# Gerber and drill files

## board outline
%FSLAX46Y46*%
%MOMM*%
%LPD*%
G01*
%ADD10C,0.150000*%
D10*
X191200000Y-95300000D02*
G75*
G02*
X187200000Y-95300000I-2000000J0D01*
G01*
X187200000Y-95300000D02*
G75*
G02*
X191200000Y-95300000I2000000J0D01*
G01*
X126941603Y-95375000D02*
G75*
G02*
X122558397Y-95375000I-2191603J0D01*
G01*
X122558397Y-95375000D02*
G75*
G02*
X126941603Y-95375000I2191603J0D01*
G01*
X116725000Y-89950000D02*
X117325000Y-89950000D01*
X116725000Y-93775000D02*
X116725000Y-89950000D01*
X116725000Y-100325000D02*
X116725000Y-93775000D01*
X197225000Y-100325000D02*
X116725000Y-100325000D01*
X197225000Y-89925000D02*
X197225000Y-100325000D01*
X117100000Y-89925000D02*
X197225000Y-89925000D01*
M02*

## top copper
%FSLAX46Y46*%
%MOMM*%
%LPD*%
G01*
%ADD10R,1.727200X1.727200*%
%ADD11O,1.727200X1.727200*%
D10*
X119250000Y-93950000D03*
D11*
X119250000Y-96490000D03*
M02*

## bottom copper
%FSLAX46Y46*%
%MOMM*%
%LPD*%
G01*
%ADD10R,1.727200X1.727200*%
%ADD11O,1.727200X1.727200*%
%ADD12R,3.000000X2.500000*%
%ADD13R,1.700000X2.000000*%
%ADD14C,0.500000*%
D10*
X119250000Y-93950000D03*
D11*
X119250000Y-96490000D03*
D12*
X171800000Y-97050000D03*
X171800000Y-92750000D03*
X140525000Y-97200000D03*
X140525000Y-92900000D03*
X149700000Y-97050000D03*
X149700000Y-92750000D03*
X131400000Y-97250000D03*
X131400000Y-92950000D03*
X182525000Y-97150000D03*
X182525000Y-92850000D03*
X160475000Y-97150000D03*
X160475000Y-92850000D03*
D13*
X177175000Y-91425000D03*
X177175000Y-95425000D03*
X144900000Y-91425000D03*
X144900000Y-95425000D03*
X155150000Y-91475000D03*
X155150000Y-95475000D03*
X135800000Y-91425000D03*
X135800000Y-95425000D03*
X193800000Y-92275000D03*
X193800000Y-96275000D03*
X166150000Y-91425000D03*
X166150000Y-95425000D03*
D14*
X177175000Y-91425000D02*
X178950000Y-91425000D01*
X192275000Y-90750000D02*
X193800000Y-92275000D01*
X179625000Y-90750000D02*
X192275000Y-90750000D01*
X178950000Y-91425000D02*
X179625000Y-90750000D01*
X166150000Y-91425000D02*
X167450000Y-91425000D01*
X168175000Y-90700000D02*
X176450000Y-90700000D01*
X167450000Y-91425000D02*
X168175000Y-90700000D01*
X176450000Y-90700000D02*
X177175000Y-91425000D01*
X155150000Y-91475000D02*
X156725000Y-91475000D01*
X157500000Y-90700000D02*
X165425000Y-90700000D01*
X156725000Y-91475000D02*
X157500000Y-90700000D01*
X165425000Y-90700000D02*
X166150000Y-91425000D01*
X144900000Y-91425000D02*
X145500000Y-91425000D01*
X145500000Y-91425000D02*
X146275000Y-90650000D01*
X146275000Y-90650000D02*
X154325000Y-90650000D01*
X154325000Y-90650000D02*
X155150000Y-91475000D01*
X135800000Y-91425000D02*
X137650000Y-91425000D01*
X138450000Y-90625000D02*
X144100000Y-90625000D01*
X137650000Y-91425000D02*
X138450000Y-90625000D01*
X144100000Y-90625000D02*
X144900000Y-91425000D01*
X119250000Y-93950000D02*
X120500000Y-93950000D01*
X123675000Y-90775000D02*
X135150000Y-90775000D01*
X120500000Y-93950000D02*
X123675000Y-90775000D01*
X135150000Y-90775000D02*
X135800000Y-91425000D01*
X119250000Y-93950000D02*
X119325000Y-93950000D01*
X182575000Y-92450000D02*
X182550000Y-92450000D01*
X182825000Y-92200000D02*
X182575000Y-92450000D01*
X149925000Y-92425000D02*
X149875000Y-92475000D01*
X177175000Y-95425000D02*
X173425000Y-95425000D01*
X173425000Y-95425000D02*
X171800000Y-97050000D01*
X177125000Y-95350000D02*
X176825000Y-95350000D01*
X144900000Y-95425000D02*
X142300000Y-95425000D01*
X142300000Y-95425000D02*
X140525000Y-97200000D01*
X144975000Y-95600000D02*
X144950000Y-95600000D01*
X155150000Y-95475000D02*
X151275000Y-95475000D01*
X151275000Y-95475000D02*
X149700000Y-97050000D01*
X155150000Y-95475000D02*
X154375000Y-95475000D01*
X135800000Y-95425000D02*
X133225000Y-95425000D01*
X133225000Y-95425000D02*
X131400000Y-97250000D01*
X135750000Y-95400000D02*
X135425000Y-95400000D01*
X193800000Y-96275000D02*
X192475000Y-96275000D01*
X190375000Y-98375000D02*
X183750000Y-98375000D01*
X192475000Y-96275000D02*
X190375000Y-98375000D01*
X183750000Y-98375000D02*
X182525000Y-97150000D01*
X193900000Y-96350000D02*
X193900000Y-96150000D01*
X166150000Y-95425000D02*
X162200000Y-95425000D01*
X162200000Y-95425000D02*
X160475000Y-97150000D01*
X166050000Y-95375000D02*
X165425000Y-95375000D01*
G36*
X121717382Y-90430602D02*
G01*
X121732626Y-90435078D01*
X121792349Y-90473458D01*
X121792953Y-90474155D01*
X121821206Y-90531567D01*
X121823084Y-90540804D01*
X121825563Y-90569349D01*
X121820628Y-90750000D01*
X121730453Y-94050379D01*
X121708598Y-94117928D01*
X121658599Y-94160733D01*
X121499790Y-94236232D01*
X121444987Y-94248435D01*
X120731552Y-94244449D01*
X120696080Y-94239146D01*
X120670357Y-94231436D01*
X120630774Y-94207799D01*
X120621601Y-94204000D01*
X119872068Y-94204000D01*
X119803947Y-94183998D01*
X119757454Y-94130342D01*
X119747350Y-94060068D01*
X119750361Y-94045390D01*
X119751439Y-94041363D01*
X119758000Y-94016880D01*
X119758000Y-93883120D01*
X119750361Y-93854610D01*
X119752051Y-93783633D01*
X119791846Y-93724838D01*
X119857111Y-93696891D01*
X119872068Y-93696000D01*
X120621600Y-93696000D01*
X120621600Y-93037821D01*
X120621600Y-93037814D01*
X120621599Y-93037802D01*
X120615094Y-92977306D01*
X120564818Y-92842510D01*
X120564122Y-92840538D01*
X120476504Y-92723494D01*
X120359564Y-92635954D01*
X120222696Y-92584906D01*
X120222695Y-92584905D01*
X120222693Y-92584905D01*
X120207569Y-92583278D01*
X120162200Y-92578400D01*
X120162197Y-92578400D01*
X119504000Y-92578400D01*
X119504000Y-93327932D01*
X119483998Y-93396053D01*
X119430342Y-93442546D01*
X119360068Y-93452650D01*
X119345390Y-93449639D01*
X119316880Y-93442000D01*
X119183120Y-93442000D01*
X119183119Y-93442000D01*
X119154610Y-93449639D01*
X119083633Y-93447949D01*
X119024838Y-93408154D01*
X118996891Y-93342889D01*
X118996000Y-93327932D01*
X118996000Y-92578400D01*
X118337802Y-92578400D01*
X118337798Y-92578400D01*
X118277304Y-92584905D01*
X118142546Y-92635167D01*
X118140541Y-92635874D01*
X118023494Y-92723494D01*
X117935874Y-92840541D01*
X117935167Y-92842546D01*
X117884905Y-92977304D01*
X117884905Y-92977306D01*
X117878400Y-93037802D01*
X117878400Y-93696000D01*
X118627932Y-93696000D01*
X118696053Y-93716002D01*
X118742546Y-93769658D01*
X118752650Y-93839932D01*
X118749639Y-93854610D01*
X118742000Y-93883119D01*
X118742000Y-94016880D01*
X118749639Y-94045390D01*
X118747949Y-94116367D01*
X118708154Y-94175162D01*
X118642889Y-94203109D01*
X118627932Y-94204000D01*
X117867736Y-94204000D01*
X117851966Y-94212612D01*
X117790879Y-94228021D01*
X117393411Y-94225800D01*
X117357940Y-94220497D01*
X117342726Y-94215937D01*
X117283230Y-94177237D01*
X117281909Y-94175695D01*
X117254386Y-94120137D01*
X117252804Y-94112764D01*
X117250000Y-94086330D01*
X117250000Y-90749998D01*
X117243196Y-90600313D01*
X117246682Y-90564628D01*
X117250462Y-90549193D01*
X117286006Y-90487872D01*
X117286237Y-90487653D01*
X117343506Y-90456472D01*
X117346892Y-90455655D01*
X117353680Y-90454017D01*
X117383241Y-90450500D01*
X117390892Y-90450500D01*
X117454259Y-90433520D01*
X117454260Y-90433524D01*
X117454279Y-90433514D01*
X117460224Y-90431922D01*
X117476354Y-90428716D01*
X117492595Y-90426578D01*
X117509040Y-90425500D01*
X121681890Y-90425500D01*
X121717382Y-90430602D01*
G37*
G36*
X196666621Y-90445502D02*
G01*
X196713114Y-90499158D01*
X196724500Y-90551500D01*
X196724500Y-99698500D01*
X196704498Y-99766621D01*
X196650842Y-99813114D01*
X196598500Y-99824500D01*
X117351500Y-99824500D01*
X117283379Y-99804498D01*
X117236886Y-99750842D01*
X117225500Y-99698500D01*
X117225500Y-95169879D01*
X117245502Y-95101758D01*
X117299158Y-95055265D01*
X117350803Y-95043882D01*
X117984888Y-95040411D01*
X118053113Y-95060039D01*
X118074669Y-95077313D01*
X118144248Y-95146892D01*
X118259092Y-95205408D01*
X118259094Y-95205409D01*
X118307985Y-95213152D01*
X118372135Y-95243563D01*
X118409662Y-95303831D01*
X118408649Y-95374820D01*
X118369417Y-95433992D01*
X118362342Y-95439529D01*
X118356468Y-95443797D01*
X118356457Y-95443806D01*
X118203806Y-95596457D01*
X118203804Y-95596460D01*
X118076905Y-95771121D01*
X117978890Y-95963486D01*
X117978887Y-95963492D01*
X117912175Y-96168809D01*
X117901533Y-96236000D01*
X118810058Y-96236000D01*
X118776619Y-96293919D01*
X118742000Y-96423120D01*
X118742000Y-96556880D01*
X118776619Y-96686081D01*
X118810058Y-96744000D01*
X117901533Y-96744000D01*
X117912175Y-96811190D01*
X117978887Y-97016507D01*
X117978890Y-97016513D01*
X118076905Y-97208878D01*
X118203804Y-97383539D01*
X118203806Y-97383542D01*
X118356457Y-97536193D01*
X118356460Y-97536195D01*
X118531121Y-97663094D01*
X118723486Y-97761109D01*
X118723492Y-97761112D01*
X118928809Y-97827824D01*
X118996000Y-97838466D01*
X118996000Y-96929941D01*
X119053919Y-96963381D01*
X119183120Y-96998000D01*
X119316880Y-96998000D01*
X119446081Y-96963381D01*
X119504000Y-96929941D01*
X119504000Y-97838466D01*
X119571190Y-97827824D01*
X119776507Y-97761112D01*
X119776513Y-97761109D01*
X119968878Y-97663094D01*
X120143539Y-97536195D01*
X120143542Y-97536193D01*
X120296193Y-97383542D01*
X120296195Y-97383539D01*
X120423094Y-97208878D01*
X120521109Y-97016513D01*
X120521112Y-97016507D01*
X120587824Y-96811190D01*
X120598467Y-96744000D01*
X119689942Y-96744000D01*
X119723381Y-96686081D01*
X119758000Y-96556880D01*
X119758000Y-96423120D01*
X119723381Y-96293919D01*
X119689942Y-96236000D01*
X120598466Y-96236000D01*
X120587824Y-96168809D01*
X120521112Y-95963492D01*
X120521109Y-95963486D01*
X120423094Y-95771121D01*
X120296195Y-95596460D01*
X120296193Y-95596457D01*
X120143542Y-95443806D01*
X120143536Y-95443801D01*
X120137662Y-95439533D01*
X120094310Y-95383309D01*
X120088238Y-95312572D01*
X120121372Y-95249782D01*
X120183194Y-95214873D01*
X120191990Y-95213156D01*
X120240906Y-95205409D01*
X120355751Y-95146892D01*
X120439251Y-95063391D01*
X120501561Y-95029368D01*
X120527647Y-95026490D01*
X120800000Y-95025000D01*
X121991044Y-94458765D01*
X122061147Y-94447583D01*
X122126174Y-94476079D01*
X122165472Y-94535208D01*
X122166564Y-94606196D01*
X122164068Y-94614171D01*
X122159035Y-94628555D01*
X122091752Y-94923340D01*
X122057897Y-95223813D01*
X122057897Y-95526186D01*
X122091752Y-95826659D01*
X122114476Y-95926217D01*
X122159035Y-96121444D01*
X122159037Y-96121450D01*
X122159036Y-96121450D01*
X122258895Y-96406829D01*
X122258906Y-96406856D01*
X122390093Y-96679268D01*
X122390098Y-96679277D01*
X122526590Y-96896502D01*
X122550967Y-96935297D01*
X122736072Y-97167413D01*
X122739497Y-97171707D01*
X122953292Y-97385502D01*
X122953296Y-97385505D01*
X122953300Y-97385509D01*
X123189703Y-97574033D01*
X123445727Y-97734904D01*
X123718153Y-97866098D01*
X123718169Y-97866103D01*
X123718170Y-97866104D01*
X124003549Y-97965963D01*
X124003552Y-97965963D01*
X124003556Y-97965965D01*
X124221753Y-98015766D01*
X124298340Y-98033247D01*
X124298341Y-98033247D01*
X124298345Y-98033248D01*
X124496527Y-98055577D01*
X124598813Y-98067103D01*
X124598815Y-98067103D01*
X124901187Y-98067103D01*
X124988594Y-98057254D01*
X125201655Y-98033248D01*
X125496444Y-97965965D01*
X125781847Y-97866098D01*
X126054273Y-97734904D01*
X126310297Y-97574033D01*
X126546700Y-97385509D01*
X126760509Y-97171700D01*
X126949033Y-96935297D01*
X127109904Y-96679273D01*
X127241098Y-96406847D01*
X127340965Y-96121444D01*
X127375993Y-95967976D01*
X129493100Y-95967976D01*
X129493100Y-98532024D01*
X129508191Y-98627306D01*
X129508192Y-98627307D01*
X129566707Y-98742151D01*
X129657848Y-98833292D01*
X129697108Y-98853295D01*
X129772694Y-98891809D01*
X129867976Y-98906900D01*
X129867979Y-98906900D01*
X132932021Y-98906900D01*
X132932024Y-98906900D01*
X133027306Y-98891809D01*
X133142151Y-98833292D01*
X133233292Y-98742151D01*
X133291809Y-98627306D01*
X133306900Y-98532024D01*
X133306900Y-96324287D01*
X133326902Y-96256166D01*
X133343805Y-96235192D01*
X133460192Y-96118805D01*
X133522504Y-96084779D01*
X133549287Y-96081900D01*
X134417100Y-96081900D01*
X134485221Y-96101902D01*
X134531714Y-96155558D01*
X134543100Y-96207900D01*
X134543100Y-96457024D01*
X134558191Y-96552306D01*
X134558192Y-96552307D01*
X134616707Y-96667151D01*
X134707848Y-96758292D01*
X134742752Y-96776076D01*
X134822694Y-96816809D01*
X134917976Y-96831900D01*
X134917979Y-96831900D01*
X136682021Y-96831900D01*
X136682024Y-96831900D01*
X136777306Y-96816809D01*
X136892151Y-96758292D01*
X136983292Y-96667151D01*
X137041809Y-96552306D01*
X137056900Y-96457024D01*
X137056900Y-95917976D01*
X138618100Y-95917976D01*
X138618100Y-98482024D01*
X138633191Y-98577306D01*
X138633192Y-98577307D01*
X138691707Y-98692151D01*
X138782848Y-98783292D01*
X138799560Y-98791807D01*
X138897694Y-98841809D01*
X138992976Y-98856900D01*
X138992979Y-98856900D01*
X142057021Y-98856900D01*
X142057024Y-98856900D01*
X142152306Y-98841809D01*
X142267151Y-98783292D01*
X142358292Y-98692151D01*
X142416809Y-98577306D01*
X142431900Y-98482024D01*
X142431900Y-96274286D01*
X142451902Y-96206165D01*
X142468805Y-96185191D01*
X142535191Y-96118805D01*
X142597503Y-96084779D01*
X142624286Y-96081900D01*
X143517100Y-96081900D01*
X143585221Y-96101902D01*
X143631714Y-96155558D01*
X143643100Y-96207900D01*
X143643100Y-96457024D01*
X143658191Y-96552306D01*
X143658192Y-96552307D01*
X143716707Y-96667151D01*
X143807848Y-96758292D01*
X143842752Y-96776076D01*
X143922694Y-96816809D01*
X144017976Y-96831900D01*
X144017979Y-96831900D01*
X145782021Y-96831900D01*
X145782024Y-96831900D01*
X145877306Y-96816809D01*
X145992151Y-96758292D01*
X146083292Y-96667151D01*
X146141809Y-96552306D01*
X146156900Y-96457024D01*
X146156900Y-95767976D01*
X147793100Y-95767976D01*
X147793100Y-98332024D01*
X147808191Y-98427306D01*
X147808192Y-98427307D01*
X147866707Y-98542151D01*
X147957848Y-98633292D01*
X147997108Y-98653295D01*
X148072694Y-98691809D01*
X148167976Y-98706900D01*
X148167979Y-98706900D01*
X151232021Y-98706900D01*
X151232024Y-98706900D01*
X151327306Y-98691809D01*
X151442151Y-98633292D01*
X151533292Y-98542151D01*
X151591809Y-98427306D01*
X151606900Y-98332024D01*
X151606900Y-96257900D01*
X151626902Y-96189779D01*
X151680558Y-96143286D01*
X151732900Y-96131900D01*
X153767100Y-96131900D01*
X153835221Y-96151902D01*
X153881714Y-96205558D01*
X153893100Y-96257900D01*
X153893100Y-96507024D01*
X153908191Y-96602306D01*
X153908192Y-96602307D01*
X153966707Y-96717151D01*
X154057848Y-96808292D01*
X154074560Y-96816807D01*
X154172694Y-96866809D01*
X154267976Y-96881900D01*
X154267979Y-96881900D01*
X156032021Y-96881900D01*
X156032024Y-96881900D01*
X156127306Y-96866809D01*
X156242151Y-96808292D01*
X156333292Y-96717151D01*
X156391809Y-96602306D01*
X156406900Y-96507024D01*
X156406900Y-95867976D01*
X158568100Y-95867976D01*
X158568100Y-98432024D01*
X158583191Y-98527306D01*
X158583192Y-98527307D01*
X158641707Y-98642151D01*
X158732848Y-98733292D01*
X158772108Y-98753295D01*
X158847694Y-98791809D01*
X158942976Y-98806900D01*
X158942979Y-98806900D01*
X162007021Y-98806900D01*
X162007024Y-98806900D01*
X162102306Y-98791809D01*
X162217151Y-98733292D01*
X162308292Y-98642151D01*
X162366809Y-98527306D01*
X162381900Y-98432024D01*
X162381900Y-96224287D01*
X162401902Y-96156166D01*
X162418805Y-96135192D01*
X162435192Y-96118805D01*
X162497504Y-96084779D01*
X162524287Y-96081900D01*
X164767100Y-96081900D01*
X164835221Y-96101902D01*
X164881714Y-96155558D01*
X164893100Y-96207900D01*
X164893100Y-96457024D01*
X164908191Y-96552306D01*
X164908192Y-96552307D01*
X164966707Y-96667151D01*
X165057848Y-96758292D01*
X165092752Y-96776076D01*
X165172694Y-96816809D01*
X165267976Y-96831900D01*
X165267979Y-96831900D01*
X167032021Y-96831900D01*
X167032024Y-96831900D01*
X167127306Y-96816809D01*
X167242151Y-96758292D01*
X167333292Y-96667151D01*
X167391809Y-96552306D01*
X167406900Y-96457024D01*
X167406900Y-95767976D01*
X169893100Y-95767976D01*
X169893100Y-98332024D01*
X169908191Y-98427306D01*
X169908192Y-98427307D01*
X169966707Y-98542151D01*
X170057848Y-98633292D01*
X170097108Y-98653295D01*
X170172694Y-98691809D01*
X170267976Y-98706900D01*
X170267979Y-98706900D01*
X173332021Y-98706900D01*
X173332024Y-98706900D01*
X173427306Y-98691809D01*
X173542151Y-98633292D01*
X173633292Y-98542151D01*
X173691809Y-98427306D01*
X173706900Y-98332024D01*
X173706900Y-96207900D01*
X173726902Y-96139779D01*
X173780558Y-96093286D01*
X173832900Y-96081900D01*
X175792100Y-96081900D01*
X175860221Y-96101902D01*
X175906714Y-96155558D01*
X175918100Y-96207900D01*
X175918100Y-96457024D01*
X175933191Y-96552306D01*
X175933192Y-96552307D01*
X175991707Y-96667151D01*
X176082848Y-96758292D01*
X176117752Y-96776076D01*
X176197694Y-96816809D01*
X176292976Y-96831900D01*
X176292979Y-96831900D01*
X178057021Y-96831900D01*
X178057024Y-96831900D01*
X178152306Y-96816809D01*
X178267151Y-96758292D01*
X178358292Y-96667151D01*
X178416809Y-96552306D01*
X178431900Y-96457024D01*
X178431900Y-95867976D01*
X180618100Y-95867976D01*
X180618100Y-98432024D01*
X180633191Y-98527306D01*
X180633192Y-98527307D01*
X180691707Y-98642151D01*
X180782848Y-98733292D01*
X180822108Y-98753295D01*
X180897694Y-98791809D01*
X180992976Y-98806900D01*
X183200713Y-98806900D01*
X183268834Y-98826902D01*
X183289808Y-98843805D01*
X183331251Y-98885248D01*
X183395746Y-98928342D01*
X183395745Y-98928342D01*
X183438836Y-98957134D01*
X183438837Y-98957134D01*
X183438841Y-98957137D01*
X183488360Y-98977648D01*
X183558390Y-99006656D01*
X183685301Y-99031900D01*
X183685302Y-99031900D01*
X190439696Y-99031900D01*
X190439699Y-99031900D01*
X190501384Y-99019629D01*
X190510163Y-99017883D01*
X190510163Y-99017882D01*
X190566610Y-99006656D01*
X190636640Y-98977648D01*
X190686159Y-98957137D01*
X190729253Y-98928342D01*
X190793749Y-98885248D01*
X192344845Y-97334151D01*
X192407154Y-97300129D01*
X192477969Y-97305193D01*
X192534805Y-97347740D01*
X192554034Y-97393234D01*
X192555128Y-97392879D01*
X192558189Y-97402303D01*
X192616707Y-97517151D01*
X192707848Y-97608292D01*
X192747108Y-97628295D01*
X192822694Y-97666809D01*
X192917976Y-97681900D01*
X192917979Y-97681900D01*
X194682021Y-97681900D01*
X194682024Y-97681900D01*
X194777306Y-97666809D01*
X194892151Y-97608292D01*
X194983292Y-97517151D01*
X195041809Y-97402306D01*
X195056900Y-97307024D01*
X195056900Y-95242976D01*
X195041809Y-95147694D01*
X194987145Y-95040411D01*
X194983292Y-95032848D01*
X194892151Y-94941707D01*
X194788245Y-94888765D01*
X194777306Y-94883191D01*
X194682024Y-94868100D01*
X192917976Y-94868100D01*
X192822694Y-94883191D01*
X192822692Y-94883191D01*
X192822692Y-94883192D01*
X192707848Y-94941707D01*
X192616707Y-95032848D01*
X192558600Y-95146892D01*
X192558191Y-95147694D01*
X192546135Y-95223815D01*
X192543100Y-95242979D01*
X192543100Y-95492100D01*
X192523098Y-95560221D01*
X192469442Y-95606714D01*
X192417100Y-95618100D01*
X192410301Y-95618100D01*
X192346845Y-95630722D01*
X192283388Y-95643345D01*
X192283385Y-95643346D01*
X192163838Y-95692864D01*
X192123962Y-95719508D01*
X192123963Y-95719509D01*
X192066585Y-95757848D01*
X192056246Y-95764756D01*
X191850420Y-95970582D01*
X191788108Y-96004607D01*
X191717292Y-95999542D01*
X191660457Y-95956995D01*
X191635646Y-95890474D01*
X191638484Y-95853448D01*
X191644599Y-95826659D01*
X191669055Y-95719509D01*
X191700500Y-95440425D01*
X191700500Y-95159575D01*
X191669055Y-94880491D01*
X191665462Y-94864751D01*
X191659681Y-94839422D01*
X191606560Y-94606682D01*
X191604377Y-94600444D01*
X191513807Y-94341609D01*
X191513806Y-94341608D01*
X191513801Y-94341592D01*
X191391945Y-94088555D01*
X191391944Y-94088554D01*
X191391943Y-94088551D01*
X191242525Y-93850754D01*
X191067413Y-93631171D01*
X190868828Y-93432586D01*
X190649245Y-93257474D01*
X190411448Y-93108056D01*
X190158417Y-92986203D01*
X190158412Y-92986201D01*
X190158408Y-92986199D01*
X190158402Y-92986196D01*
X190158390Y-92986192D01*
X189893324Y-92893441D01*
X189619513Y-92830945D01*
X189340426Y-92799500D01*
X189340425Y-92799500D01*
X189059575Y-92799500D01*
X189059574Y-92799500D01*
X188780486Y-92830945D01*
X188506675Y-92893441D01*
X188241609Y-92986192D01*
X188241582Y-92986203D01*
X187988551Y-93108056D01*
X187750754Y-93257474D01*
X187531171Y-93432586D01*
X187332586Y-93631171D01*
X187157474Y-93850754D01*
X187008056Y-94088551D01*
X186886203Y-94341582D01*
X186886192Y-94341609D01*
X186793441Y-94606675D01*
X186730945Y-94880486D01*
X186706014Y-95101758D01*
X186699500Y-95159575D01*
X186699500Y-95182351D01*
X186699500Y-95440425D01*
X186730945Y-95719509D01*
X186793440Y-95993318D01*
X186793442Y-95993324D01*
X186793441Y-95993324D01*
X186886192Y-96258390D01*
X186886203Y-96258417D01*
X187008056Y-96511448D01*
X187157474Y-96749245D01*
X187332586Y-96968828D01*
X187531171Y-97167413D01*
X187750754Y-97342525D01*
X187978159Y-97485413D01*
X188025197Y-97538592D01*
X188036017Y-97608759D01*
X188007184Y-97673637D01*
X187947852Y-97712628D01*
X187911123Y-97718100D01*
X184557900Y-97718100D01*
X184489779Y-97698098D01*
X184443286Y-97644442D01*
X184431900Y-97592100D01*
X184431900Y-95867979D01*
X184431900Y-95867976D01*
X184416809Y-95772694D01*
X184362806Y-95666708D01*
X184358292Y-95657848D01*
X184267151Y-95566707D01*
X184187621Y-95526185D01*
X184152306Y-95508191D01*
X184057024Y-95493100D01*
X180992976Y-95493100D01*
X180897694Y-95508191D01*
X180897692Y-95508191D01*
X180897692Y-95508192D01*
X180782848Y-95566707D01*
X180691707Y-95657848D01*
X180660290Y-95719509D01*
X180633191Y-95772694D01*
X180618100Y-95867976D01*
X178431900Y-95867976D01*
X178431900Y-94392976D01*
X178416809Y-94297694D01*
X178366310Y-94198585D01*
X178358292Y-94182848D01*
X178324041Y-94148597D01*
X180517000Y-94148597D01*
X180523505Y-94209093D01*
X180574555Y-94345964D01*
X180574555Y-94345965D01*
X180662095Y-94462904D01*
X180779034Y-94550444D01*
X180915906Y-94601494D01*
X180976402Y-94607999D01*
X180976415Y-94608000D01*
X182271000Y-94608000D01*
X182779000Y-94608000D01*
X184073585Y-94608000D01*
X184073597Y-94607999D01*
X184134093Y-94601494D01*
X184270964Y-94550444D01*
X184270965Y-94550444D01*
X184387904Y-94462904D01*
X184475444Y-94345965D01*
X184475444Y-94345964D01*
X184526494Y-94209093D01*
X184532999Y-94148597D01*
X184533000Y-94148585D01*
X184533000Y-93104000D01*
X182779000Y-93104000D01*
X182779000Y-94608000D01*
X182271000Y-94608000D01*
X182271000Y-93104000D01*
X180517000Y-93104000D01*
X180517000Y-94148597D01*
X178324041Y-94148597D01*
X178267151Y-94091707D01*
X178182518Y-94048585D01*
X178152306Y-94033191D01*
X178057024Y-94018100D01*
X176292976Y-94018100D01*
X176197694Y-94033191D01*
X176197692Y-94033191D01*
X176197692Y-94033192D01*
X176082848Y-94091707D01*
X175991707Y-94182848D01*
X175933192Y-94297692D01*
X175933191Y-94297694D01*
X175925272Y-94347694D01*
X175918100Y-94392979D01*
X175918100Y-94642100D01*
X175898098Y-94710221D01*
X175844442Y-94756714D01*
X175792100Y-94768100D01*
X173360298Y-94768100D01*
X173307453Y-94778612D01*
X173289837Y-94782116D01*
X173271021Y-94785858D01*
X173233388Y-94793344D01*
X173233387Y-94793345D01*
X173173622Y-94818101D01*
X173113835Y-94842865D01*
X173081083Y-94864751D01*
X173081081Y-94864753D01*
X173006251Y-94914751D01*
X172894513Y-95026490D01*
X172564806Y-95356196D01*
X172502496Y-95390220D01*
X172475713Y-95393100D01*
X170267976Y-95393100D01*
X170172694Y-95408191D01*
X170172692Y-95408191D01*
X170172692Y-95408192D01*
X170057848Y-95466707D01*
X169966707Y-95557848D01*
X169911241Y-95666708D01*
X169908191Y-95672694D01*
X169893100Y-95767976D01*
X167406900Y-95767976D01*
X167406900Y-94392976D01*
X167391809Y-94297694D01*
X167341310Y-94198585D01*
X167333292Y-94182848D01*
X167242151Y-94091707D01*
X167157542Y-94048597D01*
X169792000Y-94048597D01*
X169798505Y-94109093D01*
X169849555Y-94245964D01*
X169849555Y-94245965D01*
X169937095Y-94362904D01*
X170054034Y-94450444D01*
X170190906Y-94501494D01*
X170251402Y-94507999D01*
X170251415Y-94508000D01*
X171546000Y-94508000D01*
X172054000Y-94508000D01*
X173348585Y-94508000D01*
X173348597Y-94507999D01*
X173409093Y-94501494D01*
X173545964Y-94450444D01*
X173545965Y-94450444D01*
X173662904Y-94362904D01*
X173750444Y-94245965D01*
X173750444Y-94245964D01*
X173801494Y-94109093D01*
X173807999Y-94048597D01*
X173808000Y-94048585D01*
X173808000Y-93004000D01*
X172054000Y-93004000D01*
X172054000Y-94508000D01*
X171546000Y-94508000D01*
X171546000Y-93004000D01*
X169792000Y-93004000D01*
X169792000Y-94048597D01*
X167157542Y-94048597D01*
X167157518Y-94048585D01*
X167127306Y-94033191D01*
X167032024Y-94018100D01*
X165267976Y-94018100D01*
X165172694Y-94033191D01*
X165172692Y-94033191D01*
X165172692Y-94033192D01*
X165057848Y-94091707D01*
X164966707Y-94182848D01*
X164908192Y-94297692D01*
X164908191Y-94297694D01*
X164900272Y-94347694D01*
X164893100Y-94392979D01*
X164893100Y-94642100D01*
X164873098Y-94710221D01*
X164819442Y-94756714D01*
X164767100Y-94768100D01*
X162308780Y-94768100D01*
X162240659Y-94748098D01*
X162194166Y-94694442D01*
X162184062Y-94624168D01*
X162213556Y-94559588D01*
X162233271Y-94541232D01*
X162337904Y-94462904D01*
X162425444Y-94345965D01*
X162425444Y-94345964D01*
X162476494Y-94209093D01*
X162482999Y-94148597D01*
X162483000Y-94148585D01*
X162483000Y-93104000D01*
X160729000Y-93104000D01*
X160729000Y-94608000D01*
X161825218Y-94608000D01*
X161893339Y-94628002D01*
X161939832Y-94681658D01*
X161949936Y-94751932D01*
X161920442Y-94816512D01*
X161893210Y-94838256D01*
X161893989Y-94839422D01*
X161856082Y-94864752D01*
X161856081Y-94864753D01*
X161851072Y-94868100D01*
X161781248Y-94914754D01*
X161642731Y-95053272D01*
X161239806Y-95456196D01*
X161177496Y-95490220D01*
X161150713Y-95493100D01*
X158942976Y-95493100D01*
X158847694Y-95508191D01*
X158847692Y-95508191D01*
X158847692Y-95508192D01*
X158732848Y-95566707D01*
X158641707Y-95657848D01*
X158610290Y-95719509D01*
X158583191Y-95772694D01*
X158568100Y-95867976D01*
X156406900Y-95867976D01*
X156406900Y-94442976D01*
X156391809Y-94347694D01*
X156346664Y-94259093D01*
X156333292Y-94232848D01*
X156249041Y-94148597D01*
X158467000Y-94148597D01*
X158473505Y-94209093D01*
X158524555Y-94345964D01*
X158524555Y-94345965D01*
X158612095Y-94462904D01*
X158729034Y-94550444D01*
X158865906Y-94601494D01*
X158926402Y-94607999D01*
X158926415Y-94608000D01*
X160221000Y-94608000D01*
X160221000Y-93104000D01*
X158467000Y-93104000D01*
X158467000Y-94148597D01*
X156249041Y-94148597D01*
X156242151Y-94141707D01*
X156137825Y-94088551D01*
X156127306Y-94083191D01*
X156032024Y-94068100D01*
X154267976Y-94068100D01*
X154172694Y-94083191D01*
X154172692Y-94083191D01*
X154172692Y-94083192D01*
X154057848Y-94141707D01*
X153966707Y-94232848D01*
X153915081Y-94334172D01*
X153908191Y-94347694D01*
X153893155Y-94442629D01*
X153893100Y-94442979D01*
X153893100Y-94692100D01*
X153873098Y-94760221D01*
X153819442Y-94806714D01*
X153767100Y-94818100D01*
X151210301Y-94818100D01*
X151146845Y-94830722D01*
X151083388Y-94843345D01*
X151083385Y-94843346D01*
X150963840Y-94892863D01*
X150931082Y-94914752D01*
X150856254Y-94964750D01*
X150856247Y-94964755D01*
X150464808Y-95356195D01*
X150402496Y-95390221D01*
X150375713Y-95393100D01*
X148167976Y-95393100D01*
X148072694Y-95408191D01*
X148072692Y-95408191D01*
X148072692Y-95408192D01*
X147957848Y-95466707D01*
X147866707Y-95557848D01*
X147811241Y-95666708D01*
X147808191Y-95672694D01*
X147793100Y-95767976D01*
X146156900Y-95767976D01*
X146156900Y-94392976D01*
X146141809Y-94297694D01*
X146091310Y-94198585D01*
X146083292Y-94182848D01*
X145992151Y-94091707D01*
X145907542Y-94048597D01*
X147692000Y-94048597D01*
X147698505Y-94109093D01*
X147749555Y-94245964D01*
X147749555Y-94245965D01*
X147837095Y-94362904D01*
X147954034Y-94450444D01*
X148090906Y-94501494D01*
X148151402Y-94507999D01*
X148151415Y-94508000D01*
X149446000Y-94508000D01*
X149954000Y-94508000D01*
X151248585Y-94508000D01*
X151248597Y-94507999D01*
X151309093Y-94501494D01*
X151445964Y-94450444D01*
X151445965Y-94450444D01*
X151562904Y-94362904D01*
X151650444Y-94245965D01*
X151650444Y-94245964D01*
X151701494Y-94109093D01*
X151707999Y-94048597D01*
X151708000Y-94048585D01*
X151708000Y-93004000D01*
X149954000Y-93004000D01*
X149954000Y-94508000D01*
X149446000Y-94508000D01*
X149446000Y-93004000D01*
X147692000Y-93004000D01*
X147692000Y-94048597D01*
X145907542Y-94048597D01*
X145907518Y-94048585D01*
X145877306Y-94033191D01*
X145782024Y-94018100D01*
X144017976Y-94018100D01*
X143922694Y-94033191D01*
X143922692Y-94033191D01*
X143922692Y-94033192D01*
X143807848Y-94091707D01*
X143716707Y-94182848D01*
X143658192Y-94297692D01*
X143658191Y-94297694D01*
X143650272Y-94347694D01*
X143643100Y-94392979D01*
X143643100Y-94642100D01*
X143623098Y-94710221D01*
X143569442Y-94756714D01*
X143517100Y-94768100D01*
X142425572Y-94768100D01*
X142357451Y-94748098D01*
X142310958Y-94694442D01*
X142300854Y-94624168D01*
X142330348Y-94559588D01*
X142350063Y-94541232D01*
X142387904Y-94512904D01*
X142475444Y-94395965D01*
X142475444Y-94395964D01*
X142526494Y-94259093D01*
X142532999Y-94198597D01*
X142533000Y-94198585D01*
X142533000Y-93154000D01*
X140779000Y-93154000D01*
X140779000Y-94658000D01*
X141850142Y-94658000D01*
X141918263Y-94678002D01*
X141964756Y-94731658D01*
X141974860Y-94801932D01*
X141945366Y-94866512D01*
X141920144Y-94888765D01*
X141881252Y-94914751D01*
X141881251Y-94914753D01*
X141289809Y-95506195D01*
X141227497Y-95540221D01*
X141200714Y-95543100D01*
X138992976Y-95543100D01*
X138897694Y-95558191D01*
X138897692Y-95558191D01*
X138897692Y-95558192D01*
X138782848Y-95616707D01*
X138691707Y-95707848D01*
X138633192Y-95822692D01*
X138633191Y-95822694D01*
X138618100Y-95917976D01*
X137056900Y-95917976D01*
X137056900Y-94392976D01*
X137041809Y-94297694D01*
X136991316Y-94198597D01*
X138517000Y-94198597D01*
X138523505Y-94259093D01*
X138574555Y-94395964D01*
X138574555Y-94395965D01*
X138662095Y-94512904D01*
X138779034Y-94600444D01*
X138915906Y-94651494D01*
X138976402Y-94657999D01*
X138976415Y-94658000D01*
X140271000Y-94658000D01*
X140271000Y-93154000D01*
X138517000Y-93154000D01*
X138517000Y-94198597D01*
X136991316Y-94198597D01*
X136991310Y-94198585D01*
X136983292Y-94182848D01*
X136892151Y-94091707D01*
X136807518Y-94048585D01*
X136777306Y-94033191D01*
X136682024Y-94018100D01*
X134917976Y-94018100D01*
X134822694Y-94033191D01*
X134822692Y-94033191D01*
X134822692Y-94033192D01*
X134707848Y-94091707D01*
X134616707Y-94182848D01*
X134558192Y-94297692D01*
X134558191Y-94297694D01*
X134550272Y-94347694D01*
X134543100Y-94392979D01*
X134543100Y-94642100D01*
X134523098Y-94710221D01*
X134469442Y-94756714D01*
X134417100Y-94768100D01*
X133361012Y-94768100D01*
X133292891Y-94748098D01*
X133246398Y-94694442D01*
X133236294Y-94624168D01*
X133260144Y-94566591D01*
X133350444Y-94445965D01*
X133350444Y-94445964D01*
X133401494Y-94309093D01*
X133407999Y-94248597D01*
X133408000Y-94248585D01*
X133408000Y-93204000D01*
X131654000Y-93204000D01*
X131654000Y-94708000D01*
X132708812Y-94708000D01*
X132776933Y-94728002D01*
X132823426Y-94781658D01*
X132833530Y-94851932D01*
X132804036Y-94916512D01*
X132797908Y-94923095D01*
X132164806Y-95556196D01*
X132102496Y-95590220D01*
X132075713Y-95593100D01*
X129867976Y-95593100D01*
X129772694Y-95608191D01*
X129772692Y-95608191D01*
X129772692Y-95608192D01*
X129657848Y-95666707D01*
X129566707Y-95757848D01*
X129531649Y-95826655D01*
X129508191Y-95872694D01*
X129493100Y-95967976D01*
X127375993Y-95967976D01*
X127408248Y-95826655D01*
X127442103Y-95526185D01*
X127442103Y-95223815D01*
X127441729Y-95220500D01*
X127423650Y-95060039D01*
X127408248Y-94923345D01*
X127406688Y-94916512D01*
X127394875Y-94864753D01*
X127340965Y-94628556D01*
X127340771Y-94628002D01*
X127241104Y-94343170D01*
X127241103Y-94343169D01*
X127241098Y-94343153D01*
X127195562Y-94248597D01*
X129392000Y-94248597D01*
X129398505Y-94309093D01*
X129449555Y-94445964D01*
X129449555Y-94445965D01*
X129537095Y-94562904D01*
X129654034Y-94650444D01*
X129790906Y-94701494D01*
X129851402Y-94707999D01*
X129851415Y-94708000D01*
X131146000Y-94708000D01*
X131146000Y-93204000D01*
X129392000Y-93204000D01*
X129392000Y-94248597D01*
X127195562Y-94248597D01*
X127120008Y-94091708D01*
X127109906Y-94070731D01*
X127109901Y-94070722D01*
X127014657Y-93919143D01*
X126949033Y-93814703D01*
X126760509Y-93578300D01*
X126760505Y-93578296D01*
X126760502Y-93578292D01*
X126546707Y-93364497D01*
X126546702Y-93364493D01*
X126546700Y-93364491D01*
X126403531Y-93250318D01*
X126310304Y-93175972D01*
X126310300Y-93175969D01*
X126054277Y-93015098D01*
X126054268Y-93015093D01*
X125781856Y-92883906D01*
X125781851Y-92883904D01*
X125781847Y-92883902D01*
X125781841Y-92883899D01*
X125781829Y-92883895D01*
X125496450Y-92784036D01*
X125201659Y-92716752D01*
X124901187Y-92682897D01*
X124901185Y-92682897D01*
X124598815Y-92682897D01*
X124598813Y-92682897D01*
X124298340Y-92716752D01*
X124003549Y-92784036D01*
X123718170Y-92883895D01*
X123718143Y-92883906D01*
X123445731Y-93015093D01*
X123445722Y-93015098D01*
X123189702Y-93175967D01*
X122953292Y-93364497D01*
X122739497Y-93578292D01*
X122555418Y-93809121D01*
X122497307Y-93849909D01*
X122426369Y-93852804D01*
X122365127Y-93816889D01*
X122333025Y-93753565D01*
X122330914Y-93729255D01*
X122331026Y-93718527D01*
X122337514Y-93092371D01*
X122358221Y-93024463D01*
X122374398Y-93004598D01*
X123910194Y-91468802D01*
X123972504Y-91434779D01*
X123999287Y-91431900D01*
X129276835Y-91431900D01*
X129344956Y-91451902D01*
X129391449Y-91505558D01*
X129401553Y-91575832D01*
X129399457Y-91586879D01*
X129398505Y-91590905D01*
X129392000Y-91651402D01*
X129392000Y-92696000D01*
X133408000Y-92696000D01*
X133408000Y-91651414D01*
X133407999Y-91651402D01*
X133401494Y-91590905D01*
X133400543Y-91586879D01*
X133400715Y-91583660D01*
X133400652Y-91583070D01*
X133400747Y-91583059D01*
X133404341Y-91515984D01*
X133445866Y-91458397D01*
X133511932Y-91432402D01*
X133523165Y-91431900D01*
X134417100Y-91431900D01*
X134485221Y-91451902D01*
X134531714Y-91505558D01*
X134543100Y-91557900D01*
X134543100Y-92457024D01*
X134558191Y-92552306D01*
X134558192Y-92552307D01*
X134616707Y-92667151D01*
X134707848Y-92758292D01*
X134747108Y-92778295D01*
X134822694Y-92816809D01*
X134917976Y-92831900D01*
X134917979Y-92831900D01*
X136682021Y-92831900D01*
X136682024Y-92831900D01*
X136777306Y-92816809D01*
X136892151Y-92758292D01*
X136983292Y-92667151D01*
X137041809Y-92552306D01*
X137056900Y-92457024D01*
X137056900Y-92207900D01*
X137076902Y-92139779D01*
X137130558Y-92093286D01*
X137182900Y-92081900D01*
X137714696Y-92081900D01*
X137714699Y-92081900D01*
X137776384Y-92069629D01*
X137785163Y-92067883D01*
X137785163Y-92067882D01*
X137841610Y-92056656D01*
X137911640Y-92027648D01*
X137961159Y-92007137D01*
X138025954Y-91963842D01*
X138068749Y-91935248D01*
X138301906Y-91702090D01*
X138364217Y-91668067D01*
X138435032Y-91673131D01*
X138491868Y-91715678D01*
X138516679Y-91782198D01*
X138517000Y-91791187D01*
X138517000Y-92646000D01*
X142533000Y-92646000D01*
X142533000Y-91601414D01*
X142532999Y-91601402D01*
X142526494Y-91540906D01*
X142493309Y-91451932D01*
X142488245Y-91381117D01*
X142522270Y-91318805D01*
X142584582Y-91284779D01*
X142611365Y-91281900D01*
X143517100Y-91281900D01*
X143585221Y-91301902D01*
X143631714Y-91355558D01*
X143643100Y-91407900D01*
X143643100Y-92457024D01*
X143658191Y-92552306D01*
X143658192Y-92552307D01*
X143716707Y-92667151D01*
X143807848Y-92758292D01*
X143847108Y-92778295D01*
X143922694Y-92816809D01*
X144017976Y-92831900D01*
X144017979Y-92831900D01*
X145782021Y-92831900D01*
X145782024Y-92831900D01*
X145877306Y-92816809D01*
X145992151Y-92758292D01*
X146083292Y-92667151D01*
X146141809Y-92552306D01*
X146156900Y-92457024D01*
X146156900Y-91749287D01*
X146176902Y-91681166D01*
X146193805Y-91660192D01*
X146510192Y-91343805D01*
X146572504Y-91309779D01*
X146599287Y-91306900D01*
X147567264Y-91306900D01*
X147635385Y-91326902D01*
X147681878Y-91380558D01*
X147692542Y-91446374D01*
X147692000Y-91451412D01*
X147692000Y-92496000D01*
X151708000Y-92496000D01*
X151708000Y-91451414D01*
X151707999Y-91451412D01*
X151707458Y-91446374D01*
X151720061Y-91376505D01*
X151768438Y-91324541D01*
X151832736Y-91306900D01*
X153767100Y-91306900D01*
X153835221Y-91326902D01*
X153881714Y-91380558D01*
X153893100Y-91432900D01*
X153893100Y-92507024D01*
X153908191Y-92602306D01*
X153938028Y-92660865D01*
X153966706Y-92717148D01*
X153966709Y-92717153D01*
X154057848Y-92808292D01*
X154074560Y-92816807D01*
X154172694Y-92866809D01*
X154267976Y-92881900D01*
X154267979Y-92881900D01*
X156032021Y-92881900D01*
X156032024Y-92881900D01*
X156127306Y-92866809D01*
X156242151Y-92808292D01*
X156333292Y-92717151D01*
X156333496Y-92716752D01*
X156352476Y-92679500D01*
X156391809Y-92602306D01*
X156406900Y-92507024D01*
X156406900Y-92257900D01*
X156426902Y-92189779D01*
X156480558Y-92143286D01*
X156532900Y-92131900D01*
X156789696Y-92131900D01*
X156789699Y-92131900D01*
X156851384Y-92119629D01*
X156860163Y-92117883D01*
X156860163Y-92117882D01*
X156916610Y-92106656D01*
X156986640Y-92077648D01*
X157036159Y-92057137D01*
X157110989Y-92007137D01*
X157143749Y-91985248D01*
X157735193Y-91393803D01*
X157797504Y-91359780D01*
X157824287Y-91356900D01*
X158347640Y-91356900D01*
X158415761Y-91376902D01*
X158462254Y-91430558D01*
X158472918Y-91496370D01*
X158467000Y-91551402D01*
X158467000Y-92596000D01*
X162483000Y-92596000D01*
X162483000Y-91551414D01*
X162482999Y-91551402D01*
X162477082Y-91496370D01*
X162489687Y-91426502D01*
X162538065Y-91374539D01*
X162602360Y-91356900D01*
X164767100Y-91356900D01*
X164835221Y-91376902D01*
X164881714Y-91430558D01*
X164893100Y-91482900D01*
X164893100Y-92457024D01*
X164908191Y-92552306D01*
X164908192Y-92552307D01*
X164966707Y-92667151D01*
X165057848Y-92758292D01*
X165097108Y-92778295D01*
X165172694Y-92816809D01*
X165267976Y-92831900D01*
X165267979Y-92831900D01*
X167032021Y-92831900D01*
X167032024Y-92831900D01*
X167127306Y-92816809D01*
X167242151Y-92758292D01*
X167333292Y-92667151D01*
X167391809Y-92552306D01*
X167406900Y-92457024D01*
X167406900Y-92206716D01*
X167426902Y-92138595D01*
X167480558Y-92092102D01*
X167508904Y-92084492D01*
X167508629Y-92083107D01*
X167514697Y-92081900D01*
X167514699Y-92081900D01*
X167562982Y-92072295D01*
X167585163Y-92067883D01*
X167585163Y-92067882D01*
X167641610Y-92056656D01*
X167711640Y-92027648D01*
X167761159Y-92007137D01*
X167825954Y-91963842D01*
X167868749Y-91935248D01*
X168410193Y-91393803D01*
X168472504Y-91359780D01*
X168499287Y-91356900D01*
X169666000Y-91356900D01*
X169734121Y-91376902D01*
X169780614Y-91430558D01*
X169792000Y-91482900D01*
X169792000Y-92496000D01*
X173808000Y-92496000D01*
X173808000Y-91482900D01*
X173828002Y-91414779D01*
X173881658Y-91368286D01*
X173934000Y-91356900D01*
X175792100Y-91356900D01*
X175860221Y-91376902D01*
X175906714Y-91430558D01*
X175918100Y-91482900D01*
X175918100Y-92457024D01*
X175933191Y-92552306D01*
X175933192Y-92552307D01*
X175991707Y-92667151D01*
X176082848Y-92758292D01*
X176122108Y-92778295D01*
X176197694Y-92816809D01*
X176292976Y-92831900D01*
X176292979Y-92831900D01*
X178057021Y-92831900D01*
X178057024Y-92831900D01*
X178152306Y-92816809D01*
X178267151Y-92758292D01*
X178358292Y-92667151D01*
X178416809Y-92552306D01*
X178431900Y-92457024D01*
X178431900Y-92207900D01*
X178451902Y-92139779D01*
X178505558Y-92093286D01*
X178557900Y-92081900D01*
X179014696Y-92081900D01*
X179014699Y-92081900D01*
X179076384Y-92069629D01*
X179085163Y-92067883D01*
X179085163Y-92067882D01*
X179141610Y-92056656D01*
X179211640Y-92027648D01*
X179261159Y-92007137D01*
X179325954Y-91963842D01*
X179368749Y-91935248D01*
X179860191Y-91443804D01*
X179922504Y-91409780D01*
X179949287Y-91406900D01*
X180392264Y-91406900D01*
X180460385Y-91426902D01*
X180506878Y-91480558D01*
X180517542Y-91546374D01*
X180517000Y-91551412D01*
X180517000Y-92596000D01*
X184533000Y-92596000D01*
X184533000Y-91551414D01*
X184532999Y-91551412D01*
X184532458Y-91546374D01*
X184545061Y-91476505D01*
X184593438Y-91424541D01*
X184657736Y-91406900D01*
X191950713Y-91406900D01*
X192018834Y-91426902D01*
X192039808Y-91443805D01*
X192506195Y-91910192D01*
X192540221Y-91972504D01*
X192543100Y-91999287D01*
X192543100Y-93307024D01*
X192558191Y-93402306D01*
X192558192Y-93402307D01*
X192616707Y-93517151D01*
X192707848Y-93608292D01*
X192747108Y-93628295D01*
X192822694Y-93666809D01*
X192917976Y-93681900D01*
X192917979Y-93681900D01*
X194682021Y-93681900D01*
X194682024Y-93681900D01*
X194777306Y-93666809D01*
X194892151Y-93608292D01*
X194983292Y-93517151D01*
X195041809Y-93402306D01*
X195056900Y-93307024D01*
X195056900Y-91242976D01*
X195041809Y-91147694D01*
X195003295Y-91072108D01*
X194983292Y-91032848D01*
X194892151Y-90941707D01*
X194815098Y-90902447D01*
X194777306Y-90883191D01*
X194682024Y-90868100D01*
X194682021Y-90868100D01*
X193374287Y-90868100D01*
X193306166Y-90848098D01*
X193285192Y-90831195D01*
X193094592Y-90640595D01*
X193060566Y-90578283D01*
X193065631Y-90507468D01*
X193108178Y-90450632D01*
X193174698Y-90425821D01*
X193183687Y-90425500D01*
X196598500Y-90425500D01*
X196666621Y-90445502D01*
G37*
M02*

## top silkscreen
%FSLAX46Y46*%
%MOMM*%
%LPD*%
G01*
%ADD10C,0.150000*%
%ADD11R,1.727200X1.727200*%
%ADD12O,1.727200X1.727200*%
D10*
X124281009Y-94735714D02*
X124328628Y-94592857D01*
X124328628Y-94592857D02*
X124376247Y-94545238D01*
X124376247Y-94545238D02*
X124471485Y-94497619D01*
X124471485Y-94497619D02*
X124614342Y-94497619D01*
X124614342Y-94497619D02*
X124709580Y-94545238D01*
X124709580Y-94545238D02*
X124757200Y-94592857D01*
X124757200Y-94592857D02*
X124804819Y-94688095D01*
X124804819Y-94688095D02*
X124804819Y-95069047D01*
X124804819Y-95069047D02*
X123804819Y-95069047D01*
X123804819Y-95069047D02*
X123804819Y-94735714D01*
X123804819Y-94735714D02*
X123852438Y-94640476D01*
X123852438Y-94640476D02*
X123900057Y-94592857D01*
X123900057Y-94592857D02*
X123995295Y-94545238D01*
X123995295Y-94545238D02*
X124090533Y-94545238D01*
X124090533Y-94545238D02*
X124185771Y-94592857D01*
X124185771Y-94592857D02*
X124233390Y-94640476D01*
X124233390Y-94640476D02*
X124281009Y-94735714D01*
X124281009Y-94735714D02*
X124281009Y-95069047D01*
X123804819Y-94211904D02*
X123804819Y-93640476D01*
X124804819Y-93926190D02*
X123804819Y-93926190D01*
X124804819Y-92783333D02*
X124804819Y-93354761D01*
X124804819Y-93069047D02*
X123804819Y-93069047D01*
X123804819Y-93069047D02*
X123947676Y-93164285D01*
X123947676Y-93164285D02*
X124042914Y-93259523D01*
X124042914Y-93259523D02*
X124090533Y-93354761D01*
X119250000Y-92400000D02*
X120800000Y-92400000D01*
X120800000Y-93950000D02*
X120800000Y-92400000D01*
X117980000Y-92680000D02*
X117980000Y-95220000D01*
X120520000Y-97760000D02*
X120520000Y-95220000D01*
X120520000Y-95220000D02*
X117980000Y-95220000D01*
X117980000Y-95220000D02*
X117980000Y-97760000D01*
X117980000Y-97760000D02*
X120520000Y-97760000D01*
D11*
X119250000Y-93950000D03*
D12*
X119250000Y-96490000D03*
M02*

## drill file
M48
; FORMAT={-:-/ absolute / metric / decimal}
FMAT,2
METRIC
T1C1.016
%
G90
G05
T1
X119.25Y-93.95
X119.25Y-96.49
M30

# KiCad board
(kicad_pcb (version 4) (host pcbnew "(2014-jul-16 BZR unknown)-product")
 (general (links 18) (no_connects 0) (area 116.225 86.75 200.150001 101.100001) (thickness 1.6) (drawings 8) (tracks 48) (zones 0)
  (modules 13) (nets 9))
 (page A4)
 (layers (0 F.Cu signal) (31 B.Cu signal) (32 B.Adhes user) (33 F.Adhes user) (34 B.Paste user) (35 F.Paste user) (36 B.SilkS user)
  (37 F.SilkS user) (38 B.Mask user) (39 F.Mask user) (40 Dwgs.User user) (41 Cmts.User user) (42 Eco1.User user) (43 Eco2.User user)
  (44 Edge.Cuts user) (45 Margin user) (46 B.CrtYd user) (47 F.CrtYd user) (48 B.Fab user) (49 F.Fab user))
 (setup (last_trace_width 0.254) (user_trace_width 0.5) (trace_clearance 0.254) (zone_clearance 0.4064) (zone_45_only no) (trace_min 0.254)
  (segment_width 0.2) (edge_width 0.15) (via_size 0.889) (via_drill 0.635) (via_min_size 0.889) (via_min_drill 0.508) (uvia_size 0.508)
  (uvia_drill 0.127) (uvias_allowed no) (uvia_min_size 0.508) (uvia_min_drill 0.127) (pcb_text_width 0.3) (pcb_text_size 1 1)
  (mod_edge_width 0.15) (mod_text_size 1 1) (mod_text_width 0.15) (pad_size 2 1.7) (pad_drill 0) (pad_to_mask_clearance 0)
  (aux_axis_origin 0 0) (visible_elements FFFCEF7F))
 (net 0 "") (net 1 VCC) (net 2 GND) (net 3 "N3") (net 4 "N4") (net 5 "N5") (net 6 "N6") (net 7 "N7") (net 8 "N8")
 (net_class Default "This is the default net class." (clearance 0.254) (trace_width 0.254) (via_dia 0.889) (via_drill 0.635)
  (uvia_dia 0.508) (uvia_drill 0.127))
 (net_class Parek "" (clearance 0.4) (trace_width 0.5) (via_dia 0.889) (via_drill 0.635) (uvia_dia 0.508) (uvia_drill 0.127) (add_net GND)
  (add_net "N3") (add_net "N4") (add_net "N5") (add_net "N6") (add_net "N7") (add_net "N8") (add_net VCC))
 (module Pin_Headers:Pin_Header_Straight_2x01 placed (layer F.Cu) (at 119.25 93.95 270)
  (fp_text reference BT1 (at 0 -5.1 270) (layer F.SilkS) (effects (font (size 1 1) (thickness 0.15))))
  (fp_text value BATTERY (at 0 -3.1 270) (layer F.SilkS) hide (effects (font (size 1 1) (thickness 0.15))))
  (fp_line (start -1.55 0) (end -1.55 -1.55) (layer F.SilkS) (width 0.15))
  (fp_line (start 0 -1.55) (end -1.55 -1.55) (layer F.SilkS) (width 0.15))
  (fp_line (start -1.27 1.27) (end 1.27 1.27) (layer F.SilkS) (width 0.15))
  (fp_line (start 3.81 -1.27) (end 1.27 -1.27) (layer F.SilkS) (width 0.15))
  (fp_line (start 1.27 -1.27) (end 1.27 1.27) (layer F.SilkS) (width 0.15))
  (fp_line (start 1.27 1.27) (end 3.81 1.27) (layer F.SilkS) (width 0.15))
  (fp_line (start 3.81 1.27) (end 3.81 -1.27) (layer F.SilkS) (width 0.15))
  (pad 1 thru_hole rect (at 0 0 270) (size 1.7272 1.7272) (drill 1.016) (layers *.Cu *.Mask F.SilkS) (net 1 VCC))
  (pad 2 thru_hole oval (at 2.54 0 270) (size 1.7272 1.7272) (drill 1.016) (layers *.Cu *.Mask F.SilkS) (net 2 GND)))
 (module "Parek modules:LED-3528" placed (layer B.Cu) (at 171.8 94.9 90)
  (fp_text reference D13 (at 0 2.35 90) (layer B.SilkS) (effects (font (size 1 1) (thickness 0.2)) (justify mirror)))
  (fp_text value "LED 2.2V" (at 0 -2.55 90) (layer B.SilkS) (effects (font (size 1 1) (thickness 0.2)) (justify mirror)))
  (pad 1 smd rect (at -2.15 0 90) (size 2.5 3) (layers B.Cu B.Paste B.Mask) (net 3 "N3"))
  (pad 2 smd rect (at 2.15 0 90) (size 2.5 3) (layers B.Cu B.Paste B.Mask) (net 2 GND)))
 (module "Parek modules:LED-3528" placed (layer B.Cu) (at 140.525 95.05 90)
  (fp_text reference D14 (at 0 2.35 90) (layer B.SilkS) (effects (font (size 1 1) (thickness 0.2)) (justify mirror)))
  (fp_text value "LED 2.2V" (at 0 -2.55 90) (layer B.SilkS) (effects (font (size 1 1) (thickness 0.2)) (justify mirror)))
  (pad 1 smd rect (at -2.15 0 90) (size 2.5 3) (layers B.Cu B.Paste B.Mask) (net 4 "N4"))
  (pad 2 smd rect (at 2.15 0 90) (size 2.5 3) (layers B.Cu B.Paste B.Mask) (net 2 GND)))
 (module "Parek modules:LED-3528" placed (layer B.Cu) (at 149.7 94.9 90)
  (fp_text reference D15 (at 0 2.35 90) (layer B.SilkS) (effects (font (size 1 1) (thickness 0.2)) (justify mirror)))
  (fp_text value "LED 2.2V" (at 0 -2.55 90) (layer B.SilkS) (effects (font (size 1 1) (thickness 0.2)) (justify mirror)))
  (pad 1 smd rect (at -2.15 0 90) (size 2.5 3) (layers B.Cu B.Paste B.Mask) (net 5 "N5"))
  (pad 2 smd rect (at 2.15 0 90) (size 2.5 3) (layers B.Cu B.Paste B.Mask) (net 2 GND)))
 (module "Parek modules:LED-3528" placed (layer B.Cu) (at 131.4 95.1 90)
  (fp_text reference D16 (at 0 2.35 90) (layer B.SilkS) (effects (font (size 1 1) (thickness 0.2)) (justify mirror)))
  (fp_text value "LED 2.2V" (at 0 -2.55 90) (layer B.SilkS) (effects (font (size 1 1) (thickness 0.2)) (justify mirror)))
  (pad 1 smd rect (at -2.15 0 90) (size 2.5 3) (layers B.Cu B.Paste B.Mask) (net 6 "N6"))
  (pad 2 smd rect (at 2.15 0 90) (size 2.5 3) (layers B.Cu B.Paste B.Mask) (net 2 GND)))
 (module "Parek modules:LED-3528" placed (layer B.Cu) (at 182.525 95 90)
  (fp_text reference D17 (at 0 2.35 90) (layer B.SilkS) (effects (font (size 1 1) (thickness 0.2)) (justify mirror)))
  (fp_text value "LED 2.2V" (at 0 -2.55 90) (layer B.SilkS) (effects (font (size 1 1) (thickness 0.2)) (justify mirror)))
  (pad 1 smd rect (at -2.15 0 90) (size 2.5 3) (layers B.Cu B.Paste B.Mask) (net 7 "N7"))
  (pad 2 smd rect (at 2.15 0 90) (size 2.5 3) (layers B.Cu B.Paste B.Mask) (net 2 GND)))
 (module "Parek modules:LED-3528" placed (layer B.Cu) (at 160.475 95 90)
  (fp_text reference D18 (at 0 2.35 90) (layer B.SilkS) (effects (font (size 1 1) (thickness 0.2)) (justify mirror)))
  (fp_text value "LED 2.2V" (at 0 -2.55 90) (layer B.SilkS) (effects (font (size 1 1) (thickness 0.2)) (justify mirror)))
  (pad 1 smd rect (at -2.15 0 90) (size 2.5 3) (layers B.Cu B.Paste B.Mask) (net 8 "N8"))
  (pad 2 smd rect (at 2.15 0 90) (size 2.5 3) (layers B.Cu B.Paste B.Mask) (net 2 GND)))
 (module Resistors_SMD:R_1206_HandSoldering (layer B.Cu) (at 177.175 93.425 270)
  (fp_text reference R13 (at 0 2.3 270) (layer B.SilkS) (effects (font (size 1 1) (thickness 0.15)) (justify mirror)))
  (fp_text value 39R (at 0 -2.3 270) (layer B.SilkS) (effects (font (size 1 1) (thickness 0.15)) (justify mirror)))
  (pad 1 smd rect (at -2 0 270) (size 2 1.7) (layers B.Cu B.Paste B.Mask) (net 1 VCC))
  (pad 2 smd rect (at 2 0 270) (size 2 1.7) (layers B.Cu B.Paste B.Mask) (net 3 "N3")))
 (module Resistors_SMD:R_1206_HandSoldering (layer B.Cu) (at 144.9 93.425 270)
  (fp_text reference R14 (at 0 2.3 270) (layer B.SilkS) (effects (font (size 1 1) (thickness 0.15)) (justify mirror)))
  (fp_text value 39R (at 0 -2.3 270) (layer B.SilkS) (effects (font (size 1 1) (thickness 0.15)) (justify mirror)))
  (pad 1 smd rect (at -2 0 270) (size 2 1.7) (layers B.Cu B.Paste B.Mask) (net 1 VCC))
  (pad 2 smd rect (at 2 0 270) (size 2 1.7) (layers B.Cu B.Paste B.Mask) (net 4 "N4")))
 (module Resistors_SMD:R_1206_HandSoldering (layer B.Cu) (at 155.15 93.475 270)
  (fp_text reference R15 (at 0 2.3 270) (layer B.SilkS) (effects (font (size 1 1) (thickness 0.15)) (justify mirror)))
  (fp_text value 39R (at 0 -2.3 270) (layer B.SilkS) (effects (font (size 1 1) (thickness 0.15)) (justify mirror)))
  (pad 1 smd rect (at -2 0 270) (size 2 1.7) (layers B.Cu B.Paste B.Mask) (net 1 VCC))
  (pad 2 smd rect (at 2 0 270) (size 2 1.7) (layers B.Cu B.Paste B.Mask) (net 5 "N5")))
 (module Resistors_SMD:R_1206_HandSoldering (layer B.Cu) (at 135.8 93.425 270)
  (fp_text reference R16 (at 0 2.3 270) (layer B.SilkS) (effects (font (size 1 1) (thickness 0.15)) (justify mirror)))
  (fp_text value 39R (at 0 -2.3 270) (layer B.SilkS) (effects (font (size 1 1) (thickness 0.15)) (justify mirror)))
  (pad 1 smd rect (at -2 0 270) (size 2 1.7) (layers B.Cu B.Paste B.Mask) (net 1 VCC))
  (pad 2 smd rect (at 2 0 270) (size 2 1.7) (layers B.Cu B.Paste B.Mask) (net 6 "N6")))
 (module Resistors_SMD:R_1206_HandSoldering (layer B.Cu) (at 193.8 94.275 270)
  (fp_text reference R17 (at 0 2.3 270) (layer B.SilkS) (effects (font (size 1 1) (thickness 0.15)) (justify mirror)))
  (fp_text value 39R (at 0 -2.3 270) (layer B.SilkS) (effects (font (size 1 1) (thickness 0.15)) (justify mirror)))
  (pad 1 smd rect (at -2 0 270) (size 2 1.7) (layers B.Cu B.Paste B.Mask) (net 1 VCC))
  (pad 2 smd rect (at 2 0 270) (size 2 1.7) (layers B.Cu B.Paste B.Mask) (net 7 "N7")))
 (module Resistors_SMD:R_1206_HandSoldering (layer B.Cu) (at 166.15 93.425 270)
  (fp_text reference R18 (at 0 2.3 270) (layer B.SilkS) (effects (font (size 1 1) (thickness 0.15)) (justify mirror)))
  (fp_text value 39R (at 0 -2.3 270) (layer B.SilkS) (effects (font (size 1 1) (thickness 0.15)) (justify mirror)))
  (pad 1 smd rect (at -2 0 270) (size 2 1.7) (layers B.Cu B.Paste B.Mask) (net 1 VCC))
  (pad 2 smd rect (at 2 0 270) (size 2 1.7) (layers B.Cu B.Paste B.Mask) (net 8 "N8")))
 (gr_circle (center 189.2 95.3) (end 189.2 97.3) (layer Edge.Cuts) (width 0.15))
 (gr_circle (center 124.75 95.375) (end 125.7 97.35) (layer Edge.Cuts) (width 0.15))
 (gr_line (start 116.725 89.95) (end 117.325 89.95) (angle 90) (layer Edge.Cuts) (width 0.15))
 (gr_line (start 116.725 93.775) (end 116.725 89.95) (angle 90) (layer Edge.Cuts) (width 0.15))
 (gr_line (start 116.725 100.325) (end 116.725 93.775) (angle 90) (layer Edge.Cuts) (width 0.15))
 (gr_line (start 197.225 100.325) (end 116.725 100.325) (angle 90) (layer Edge.Cuts) (width 0.15))
 (gr_line (start 197.225 89.925) (end 197.225 100.325) (angle 90) (layer Edge.Cuts) (width 0.15))
 (gr_line (start 117.1 89.925) (end 197.225 89.925) (angle 90) (layer Edge.Cuts) (width 0.15))
 (segment (start 177.175 91.425) (end 178.95 91.425) (width 0.5) (layer B.Cu) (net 1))
 (segment (start 192.275 90.75) (end 193.8 92.275) (width 0.5) (layer B.Cu) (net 1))
 (segment (start 179.625 90.75) (end 192.275 90.75) (width 0.5) (layer B.Cu) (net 1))
 (segment (start 178.95 91.425) (end 179.625 90.75) (width 0.5) (layer B.Cu) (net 1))
 (segment (start 166.15 91.425) (end 167.45 91.425) (width 0.5) (layer B.Cu) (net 1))
 (segment (start 168.175 90.7) (end 176.45 90.7) (width 0.5) (layer B.Cu) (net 1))
 (segment (start 167.45 91.425) (end 168.175 90.7) (width 0.5) (layer B.Cu) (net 1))
 (segment (start 176.45 90.7) (end 177.175 91.425) (width 0.5) (layer B.Cu) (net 1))
 (segment (start 155.15 91.475) (end 156.725 91.475) (width 0.5) (layer B.Cu) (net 1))
 (segment (start 157.5 90.7) (end 165.425 90.7) (width 0.5) (layer B.Cu) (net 1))
 (segment (start 156.725 91.475) (end 157.5 90.7) (width 0.5) (layer B.Cu) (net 1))
 (segment (start 165.425 90.7) (end 166.15 91.425) (width 0.5) (layer B.Cu) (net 1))
 (segment (start 144.9 91.425) (end 145.5 91.425) (width 0.5) (layer B.Cu) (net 1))
 (segment (start 145.5 91.425) (end 146.275 90.65) (width 0.5) (layer B.Cu) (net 1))
 (segment (start 146.275 90.65) (end 154.325 90.65) (width 0.5) (layer B.Cu) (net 1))
 (segment (start 154.325 90.65) (end 155.15 91.475) (width 0.5) (layer B.Cu) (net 1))
 (segment (start 135.8 91.425) (end 137.65 91.425) (width 0.5) (layer B.Cu) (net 1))
 (segment (start 138.45 90.625) (end 144.1 90.625) (width 0.5) (layer B.Cu) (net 1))
 (segment (start 137.65 91.425) (end 138.45 90.625) (width 0.5) (layer B.Cu) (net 1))
 (segment (start 144.1 90.625) (end 144.9 91.425) (width 0.5) (layer B.Cu) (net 1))
 (segment (start 119.25 93.95) (end 120.5 93.95) (width 0.5) (layer B.Cu) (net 1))
 (segment (start 123.675 90.775) (end 135.15 90.775) (width 0.5) (layer B.Cu) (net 1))
 (segment (start 120.5 93.95) (end 123.675 90.775) (width 0.5) (layer B.Cu) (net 1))
 (segment (start 135.15 90.775) (end 135.8 91.425) (width 0.5) (layer B.Cu) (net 1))
 (segment (start 119.25 93.95) (end 119.325 93.95) (width 0.5) (layer B.Cu) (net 1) (status 30))
 (segment (start 182.575 92.45) (end 182.55 92.45) (width 0.5) (layer B.Cu) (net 2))
 (segment (start 182.825 92.2) (end 182.575 92.45) (width 0.5) (layer B.Cu) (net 2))
 (segment (start 149.925 92.425) (end 149.875 92.475) (width 0.5) (layer B.Cu) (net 2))
 (segment (start 177.175 95.425) (end 173.425 95.425) (width 0.5) (layer B.Cu) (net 3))
 (segment (start 173.425 95.425) (end 171.8 97.05) (width 0.5) (layer B.Cu) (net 3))
 (segment (start 177.125 95.35) (end 176.825 95.35) (width 0.5) (layer B.Cu) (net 3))
 (segment (start 144.9 95.425) (end 142.3 95.425) (width 0.5) (layer B.Cu) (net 4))
 (segment (start 142.3 95.425) (end 140.525 97.2) (width 0.5) (layer B.Cu) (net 4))
 (segment (start 144.975 95.6) (end 144.95 95.6) (width 0.5) (layer B.Cu) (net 4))
 (segment (start 155.15 95.475) (end 151.275 95.475) (width 0.5) (layer B.Cu) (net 5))
 (segment (start 151.275 95.475) (end 149.7 97.05) (width 0.5) (layer B.Cu) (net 5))
 (segment (start 155.15 95.475) (end 154.375 95.475) (width 0.5) (layer B.Cu) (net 5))
 (segment (start 135.8 95.425) (end 133.225 95.425) (width 0.5) (layer B.Cu) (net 6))
 (segment (start 133.225 95.425) (end 131.4 97.25) (width 0.5) (layer B.Cu) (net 6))
 (segment (start 135.75 95.4) (end 135.425 95.4) (width 0.5) (layer B.Cu) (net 6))
 (segment (start 193.8 96.275) (end 192.475 96.275) (width 0.5) (layer B.Cu) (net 7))
 (segment (start 190.375 98.375) (end 183.75 98.375) (width 0.5) (layer B.Cu) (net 7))
 (segment (start 192.475 96.275) (end 190.375 98.375) (width 0.5) (layer B.Cu) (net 7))
 (segment (start 183.75 98.375) (end 182.525 97.15) (width 0.5) (layer B.Cu) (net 7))
 (segment (start 193.9 96.35) (end 193.9 96.15) (width 0.5) (layer B.Cu) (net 7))
 (segment (start 166.15 95.425) (end 162.2 95.425) (width 0.5) (layer B.Cu) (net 8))
 (segment (start 162.2 95.425) (end 160.475 97.15) (width 0.5) (layer B.Cu) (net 8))
 (segment (start 166.05 95.375) (end 165.425 95.375) (width 0.5) (layer B.Cu) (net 8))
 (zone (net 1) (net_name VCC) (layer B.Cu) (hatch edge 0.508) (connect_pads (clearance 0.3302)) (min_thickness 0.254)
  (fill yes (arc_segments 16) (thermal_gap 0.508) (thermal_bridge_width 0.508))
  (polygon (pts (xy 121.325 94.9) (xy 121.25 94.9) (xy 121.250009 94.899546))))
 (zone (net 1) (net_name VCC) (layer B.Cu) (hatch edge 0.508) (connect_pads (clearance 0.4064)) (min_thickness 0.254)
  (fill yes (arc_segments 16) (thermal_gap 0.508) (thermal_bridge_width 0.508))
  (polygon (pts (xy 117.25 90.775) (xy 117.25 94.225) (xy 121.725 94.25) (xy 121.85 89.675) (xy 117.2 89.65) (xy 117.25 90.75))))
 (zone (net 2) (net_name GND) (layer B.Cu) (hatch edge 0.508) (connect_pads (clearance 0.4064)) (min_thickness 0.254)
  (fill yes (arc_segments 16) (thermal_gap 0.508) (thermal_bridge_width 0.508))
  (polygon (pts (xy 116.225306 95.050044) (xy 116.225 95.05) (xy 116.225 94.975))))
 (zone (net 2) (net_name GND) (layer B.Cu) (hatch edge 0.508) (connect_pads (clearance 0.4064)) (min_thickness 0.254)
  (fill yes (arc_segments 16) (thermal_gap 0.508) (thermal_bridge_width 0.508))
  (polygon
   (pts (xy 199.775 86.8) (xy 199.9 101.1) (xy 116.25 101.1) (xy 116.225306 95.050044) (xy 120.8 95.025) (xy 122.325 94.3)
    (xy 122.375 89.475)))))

